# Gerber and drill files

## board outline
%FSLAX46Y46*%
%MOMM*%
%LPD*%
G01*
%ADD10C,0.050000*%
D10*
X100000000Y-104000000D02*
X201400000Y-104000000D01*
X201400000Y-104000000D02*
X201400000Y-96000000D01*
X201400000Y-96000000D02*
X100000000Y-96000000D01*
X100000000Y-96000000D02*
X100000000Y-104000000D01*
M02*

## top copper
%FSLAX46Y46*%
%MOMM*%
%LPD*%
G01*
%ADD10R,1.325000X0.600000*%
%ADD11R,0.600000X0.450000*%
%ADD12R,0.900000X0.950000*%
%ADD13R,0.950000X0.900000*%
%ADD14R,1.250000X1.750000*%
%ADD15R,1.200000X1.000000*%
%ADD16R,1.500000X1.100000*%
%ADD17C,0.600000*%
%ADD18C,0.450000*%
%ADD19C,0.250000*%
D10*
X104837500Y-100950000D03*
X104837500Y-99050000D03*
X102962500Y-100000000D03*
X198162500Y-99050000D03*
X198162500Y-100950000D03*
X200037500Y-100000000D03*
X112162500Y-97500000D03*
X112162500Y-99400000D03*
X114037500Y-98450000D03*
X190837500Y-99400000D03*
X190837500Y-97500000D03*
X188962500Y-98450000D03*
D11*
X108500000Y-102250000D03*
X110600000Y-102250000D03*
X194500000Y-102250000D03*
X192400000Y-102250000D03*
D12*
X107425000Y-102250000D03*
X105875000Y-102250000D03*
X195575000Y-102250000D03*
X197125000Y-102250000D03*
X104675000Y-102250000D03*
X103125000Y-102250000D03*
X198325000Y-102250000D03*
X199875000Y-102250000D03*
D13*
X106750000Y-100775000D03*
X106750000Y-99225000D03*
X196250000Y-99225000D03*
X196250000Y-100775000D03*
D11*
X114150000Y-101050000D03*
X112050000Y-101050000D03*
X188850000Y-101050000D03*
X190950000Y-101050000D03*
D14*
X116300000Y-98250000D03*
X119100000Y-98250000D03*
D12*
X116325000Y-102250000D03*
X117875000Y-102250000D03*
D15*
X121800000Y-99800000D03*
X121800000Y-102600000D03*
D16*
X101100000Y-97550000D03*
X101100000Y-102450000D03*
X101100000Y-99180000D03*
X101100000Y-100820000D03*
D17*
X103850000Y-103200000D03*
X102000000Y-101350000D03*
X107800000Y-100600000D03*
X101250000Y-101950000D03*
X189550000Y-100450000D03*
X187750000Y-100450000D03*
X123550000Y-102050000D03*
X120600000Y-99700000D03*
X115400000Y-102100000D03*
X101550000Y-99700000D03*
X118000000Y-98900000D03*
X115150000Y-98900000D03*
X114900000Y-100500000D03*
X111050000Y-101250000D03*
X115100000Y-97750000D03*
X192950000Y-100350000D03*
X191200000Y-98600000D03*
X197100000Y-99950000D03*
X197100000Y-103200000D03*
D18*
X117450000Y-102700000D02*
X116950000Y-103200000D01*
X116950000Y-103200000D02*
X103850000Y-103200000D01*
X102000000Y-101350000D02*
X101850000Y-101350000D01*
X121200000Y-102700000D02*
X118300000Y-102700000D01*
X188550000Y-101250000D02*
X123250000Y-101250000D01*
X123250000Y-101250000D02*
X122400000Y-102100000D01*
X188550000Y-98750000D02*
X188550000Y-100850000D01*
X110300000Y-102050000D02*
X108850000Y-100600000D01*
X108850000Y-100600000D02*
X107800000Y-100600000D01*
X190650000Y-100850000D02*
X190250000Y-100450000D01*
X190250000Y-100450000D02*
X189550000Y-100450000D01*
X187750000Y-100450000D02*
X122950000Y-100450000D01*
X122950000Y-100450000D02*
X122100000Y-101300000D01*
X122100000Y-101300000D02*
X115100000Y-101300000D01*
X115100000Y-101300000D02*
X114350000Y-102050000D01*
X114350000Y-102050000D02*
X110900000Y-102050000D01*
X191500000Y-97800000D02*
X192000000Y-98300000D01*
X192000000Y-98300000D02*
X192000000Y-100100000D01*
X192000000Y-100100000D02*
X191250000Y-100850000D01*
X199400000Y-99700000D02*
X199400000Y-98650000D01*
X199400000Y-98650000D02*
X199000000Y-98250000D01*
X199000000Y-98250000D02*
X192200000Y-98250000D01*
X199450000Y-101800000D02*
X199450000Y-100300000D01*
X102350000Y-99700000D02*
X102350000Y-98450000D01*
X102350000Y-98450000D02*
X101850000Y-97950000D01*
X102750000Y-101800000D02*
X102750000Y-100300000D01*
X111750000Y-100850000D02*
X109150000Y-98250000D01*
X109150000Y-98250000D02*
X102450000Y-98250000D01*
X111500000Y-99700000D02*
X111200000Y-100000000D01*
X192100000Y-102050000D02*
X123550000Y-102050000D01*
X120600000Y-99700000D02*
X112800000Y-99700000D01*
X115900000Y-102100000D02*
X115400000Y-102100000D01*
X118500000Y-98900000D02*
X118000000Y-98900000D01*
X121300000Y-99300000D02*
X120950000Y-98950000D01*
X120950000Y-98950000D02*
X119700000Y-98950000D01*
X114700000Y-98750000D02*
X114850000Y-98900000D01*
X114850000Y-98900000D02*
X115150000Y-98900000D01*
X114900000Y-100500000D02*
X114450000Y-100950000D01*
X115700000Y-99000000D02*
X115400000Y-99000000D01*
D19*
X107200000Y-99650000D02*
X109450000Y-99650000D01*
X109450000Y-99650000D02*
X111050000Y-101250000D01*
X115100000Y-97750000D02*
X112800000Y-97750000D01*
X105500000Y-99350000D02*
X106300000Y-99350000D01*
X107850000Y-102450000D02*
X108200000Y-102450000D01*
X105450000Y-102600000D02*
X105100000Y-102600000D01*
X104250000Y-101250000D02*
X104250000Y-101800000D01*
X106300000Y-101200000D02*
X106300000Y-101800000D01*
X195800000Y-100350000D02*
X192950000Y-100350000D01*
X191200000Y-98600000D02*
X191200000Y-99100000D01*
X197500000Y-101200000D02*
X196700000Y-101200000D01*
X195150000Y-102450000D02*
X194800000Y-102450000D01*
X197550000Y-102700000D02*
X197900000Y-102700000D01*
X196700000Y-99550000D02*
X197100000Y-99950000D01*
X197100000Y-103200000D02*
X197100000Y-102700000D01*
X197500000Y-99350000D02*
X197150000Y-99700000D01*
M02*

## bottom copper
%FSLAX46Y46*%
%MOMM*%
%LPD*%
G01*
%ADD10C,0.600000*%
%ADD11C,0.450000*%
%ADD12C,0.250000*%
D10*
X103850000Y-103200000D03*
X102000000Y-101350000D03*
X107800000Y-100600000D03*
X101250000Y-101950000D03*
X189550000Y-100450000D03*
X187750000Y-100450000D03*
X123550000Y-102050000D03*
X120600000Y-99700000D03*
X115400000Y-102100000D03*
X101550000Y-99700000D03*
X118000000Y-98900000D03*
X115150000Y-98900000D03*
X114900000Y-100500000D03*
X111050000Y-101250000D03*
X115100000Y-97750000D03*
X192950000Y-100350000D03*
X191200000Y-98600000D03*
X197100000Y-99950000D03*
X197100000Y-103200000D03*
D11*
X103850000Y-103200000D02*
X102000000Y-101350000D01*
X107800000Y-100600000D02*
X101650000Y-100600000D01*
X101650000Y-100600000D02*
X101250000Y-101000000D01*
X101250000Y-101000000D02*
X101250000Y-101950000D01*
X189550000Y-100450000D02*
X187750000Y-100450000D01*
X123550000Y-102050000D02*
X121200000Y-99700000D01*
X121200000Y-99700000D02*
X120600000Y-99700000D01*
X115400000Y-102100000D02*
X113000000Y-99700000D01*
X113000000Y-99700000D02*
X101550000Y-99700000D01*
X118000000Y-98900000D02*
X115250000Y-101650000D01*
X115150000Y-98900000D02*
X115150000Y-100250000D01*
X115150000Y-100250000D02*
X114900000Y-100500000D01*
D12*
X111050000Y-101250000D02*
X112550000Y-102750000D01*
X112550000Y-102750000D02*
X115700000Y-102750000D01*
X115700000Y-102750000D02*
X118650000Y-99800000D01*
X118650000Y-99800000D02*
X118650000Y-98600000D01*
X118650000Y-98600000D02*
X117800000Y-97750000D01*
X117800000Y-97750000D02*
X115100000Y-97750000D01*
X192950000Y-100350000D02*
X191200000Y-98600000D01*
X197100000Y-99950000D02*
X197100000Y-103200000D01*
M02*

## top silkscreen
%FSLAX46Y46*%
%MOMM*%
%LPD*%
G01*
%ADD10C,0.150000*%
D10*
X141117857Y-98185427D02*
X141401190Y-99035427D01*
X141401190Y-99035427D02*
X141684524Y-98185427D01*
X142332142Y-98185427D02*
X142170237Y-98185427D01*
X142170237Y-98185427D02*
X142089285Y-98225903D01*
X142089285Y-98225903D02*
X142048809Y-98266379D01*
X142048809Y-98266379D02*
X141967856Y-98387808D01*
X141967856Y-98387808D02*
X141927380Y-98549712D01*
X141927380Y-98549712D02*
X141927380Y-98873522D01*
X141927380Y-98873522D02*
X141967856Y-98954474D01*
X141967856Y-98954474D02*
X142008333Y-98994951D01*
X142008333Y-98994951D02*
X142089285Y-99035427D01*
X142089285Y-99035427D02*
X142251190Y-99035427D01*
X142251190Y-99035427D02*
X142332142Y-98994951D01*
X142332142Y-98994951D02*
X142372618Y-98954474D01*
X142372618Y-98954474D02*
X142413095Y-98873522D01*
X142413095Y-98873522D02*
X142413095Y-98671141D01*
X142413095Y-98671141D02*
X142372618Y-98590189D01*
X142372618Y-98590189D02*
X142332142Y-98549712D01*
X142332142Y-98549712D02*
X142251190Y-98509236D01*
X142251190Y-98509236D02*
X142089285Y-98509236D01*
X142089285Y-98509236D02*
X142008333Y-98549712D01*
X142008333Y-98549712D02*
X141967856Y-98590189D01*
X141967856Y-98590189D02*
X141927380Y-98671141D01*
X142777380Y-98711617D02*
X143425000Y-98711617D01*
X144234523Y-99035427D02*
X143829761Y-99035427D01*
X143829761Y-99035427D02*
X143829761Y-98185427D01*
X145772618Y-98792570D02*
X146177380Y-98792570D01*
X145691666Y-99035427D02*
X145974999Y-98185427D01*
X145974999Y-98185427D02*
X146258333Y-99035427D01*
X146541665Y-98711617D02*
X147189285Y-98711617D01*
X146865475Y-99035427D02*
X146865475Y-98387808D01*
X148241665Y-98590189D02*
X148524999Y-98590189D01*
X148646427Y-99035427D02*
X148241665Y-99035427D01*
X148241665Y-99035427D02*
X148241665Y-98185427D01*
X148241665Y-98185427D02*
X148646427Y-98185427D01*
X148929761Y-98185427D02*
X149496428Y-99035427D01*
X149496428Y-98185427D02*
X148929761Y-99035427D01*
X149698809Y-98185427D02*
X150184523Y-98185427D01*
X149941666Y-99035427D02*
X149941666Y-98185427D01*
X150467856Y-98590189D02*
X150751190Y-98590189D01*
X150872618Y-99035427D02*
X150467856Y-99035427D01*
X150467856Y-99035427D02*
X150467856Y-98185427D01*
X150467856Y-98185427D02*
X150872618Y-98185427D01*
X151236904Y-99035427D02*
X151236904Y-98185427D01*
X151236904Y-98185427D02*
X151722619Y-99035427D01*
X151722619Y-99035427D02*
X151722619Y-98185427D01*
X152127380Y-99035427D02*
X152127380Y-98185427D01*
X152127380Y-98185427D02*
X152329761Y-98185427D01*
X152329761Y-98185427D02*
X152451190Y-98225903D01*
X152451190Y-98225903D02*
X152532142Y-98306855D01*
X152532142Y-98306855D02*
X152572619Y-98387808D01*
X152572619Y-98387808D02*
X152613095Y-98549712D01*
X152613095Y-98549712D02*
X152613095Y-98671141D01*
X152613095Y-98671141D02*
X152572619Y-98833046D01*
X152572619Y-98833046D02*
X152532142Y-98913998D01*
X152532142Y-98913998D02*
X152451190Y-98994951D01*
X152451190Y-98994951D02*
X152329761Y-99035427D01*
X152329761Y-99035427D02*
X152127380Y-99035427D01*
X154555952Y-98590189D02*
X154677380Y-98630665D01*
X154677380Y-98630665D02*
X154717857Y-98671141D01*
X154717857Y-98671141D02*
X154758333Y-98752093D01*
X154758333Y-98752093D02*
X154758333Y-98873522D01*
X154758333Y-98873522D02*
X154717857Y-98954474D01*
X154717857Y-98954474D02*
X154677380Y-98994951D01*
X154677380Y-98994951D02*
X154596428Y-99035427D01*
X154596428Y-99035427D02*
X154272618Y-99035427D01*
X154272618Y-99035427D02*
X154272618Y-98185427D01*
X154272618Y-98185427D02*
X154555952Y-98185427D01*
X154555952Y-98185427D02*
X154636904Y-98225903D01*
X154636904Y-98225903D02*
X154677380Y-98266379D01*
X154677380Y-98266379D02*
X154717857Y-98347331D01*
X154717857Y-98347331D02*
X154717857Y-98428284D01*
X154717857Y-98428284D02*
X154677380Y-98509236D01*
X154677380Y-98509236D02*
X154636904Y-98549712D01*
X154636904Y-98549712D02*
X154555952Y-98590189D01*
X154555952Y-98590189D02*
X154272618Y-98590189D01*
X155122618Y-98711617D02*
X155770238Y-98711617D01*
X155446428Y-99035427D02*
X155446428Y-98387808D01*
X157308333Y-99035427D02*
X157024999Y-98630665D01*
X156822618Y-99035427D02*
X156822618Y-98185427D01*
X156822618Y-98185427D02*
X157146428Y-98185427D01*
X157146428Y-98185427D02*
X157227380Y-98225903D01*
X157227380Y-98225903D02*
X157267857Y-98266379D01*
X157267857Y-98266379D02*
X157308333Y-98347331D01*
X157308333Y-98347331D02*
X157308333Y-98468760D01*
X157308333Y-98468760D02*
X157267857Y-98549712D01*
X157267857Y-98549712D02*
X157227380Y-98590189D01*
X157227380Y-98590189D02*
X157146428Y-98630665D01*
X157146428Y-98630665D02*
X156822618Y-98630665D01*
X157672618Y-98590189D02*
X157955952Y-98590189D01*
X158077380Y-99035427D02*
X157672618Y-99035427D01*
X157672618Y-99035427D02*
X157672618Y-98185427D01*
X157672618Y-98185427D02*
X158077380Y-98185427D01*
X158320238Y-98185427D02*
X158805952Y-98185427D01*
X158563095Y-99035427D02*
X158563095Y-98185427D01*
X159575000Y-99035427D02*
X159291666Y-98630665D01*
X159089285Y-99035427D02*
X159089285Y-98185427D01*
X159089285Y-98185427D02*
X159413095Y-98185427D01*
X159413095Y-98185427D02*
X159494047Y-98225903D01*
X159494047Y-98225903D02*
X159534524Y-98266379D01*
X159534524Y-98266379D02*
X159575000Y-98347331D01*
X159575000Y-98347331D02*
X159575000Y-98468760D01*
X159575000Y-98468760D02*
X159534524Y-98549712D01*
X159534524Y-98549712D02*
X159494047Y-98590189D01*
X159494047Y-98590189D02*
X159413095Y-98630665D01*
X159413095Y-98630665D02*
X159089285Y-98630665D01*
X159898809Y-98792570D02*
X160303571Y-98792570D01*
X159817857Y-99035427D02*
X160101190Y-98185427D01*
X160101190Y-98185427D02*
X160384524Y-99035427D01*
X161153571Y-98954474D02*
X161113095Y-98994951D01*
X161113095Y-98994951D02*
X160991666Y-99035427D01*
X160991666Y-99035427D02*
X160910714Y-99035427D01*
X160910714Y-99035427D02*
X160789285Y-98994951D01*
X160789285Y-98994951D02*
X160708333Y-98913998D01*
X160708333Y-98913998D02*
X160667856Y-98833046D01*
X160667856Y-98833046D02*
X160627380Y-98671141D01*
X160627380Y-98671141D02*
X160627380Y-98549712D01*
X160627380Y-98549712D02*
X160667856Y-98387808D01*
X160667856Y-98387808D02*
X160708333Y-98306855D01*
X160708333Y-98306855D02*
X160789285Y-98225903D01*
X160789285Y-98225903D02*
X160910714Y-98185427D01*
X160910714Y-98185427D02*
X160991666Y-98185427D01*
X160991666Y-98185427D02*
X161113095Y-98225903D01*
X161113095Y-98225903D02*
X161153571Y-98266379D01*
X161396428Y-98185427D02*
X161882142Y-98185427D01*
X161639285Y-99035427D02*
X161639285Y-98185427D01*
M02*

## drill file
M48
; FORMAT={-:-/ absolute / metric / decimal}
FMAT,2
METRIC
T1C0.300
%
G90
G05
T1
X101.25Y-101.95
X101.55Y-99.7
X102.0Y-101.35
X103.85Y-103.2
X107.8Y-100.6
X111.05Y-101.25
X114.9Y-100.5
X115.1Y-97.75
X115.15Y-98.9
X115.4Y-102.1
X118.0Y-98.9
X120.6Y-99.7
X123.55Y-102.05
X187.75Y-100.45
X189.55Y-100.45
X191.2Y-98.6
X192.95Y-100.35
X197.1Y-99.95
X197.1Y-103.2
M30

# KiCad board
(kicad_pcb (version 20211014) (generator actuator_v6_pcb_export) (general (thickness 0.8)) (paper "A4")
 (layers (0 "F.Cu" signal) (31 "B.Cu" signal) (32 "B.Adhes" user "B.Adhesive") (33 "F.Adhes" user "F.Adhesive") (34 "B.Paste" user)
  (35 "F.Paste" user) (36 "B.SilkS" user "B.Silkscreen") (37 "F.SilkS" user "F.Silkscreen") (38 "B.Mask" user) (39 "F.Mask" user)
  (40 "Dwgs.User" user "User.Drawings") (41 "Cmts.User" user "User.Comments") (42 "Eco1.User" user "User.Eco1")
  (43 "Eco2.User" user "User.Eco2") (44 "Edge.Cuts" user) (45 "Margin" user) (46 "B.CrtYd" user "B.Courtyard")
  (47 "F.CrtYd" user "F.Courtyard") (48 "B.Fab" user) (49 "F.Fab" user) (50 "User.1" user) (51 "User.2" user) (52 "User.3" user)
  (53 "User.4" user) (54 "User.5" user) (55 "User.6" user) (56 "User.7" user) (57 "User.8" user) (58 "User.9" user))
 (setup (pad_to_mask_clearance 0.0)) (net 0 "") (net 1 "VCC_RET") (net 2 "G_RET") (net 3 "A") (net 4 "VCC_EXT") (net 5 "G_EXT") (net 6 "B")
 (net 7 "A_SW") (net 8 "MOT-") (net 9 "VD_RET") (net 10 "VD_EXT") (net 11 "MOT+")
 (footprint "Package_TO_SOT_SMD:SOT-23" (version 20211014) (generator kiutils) (layer "F.Cu") (at 103.9 100.0 180)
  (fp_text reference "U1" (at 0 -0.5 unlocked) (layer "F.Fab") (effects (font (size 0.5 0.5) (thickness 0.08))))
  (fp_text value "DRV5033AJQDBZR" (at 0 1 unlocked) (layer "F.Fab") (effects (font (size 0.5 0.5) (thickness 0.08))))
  (pad "1" smd rect (at -0.9375 -0.95 180) (size 1.325 0.6) (layers "F.Cu" "F.Mask" "F.Paste") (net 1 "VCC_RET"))
  (pad "2" smd rect (at -0.9375 0.95 180) (size 1.325 0.6) (layers "F.Cu" "F.Mask" "F.Paste") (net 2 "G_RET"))
  (pad "3" smd rect (at 0.9375 0.0 180) (size 1.325 0.6) (layers "F.Cu" "F.Mask" "F.Paste") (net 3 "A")))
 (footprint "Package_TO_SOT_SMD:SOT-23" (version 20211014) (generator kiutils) (layer "F.Cu") (at 199.1 100.0)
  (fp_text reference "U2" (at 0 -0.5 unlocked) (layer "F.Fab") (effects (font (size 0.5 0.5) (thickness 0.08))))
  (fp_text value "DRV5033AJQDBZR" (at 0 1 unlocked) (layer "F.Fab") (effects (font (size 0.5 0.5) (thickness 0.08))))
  (pad "1" smd rect (at -0.9375 -0.95) (size 1.325 0.6) (layers "F.Cu" "F.Mask" "F.Paste") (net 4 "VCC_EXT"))
  (pad "2" smd rect (at -0.9375 0.95) (size 1.325 0.6) (layers "F.Cu" "F.Mask" "F.Paste") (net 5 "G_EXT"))
  (pad "3" smd rect (at 0.9375 0.0) (size 1.325 0.6) (layers "F.Cu" "F.Mask" "F.Paste") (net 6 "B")))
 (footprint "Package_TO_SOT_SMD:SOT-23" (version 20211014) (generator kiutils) (layer "F.Cu") (at 113.1 98.45)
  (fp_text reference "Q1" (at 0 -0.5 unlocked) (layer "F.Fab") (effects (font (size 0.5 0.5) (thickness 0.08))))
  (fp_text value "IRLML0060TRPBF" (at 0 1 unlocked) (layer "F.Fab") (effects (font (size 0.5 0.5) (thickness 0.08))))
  (pad "1" smd rect (at -0.9375 -0.95) (size 1.325 0.6) (layers "F.Cu" "F.Mask" "F.Paste") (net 2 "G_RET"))
  (pad "2" smd rect (at -0.9375 0.95) (size 1.325 0.6) (layers "F.Cu" "F.Mask" "F.Paste") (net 3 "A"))
  (pad "3" smd rect (at 0.9375 0.0) (size 1.325 0.6) (layers "F.Cu" "F.Mask" "F.Paste") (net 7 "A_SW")))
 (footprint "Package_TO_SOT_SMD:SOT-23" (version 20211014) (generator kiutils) (layer "F.Cu") (at 189.9 98.45 180)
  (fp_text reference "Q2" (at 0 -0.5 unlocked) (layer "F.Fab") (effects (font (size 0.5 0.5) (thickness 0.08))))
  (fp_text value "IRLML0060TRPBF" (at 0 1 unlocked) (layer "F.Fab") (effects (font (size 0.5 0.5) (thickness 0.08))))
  (pad "1" smd rect (at -0.9375 -0.95 180) (size 1.325 0.6) (layers "F.Cu" "F.Mask" "F.Paste") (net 5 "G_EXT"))
  (pad "2" smd rect (at -0.9375 0.95 180) (size 1.325 0.6) (layers "F.Cu" "F.Mask" "F.Paste") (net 6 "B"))
  (pad "3" smd rect (at 0.9375 0.0 180) (size 1.325 0.6) (layers "F.Cu" "F.Mask" "F.Paste") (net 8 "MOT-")))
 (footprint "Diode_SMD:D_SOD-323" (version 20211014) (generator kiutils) (layer "F.Cu") (at 109.55 102.25)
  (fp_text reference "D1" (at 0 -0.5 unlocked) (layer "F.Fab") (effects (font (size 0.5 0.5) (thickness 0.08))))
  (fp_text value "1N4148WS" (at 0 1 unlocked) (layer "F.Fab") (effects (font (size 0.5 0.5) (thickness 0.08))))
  (pad "1" smd rect (at -1.05 0.0) (size 0.6 0.45) (layers "F.Cu" "F.Mask" "F.Paste") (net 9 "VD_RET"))
  (pad "2" smd rect (at 1.05 0.0) (size 0.6 0.45) (layers "F.Cu" "F.Mask" "F.Paste") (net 6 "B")))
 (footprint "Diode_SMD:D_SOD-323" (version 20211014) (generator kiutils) (layer "F.Cu") (at 193.45 102.25 180)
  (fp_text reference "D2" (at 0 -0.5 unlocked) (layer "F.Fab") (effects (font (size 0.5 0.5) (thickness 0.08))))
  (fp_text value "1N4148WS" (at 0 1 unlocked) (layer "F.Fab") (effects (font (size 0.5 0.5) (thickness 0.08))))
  (pad "1" smd rect (at -1.05 0.0 180) (size 0.6 0.45) (layers "F.Cu" "F.Mask" "F.Paste") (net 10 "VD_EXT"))
  (pad "2" smd rect (at 1.05 0.0 180) (size 0.6 0.45) (layers "F.Cu" "F.Mask" "F.Paste") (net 3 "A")))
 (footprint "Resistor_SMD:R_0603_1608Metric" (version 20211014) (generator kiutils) (layer "F.Cu") (at 106.65 102.25 180)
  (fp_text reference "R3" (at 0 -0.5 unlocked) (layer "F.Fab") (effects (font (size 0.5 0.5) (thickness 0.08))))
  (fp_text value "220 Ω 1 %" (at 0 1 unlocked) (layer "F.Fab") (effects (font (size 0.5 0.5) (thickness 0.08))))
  (pad "1" smd rect (at -0.775 0.0 180) (size 0.9 0.95) (layers "F.Cu" "F.Mask" "F.Paste") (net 9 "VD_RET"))
  (pad "2" smd rect (at 0.775 0.0 180) (size 0.9 0.95) (layers "F.Cu" "F.Mask" "F.Paste") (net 1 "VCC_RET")))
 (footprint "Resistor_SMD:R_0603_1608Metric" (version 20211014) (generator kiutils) (layer "F.Cu") (at 196.35 102.25)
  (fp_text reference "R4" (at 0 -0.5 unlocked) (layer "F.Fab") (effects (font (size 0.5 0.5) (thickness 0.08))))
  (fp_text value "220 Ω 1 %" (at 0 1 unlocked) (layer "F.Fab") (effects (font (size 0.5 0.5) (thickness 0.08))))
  (pad "1" smd rect (at -0.775 0.0) (size 0.9 0.95) (layers "F.Cu" "F.Mask" "F.Paste") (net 10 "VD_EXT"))
  (pad "2" smd rect (at 0.775 0.0) (size 0.9 0.95) (layers "F.Cu" "F.Mask" "F.Paste") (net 4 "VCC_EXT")))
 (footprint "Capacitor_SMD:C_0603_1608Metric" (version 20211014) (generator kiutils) (layer "F.Cu") (at 103.9 102.25 180)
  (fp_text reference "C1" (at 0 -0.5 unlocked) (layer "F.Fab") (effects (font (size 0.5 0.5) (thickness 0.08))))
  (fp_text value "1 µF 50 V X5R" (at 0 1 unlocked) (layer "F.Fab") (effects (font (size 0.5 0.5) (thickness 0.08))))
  (pad "1" smd rect (at -0.775 0.0 180) (size 0.9 0.95) (layers "F.Cu" "F.Mask" "F.Paste") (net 1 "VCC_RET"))
  (pad "2" smd rect (at 0.775 0.0 180) (size 0.9 0.95) (layers "F.Cu" "F.Mask" "F.Paste") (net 3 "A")))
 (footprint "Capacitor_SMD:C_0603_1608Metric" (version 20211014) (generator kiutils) (layer "F.Cu") (at 199.1 102.25)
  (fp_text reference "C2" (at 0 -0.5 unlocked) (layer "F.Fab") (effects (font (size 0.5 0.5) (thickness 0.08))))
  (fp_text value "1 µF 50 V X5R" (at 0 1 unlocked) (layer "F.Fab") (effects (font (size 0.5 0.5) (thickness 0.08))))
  (pad "1" smd rect (at -0.775 0.0) (size 0.9 0.95) (layers "F.Cu" "F.Mask" "F.Paste") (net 4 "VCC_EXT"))
  (pad "2" smd rect (at 0.775 0.0) (size 0.9 0.95) (layers "F.Cu" "F.Mask" "F.Paste") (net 6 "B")))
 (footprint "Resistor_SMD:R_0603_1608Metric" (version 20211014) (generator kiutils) (layer "F.Cu") (at 106.75 100.0 90)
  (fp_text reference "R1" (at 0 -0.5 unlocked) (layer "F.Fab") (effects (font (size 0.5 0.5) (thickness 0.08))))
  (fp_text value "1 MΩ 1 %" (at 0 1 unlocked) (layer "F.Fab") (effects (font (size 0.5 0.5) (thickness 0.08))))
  (pad "1" smd rect (at -0.775 0.0 90) (size 0.9 0.95) (layers "F.Cu" "F.Mask" "F.Paste") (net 1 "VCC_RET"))
  (pad "2" smd rect (at 0.775 0.0 90) (size 0.9 0.95) (layers "F.Cu" "F.Mask" "F.Paste") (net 2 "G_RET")))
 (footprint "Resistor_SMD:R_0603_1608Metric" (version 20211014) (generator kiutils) (layer "F.Cu") (at 196.25 100.0 270)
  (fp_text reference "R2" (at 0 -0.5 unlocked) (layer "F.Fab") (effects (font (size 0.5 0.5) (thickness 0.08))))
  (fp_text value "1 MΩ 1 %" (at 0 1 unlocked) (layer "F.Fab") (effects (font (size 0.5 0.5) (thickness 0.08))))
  (pad "1" smd rect (at -0.775 0.0 270) (size 0.9 0.95) (layers "F.Cu" "F.Mask" "F.Paste") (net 4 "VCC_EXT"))
  (pad "2" smd rect (at 0.775 0.0 270) (size 0.9 0.95) (layers "F.Cu" "F.Mask" "F.Paste") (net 5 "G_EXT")))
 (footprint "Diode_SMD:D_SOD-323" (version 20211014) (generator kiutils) (layer "F.Cu") (at 113.1 101.05 180)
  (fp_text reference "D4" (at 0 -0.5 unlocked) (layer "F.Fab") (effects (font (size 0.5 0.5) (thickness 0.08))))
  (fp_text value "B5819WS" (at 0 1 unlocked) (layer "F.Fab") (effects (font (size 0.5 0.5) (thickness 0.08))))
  (pad "1" smd rect (at -1.05 0.0 180) (size 0.6 0.45) (layers "F.Cu" "F.Mask" "F.Paste") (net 7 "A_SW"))
  (pad "2" smd rect (at 1.05 0.0 180) (size 0.6 0.45) (layers "F.Cu" "F.Mask" "F.Paste") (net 3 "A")))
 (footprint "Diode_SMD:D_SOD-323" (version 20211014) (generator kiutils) (layer "F.Cu") (at 189.9 101.05)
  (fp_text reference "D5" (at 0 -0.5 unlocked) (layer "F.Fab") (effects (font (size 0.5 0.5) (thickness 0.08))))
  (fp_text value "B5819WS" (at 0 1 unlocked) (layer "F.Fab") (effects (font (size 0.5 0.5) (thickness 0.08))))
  (pad "1" smd rect (at -1.05 0.0) (size 0.6 0.45) (layers "F.Cu" "F.Mask" "F.Paste") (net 8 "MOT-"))
  (pad "2" smd rect (at 1.05 0.0) (size 0.6 0.45) (layers "F.Cu" "F.Mask" "F.Paste") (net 6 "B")))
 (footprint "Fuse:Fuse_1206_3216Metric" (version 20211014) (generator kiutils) (layer "F.Cu") (at 117.7 98.25)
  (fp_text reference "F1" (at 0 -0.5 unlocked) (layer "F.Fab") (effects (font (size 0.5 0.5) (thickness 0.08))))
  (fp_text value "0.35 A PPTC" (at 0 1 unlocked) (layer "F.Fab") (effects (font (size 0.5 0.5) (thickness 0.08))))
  (pad "1" smd rect (at -1.4 0.0) (size 1.25 1.75) (layers "F.Cu" "F.Mask" "F.Paste") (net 7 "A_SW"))
  (pad "2" smd rect (at 1.4 0.0) (size 1.25 1.75) (layers "F.Cu" "F.Mask" "F.Paste") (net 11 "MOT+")))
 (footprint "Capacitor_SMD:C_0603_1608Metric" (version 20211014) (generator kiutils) (layer "F.Cu") (at 117.1 102.25)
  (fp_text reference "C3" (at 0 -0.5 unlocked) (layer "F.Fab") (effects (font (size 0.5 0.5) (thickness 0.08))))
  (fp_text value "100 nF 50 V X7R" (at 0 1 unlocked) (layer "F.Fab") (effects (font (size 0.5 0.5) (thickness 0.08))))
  (pad "1" smd rect (at -0.775 0.0) (size 0.9 0.95) (layers "F.Cu" "F.Mask" "F.Paste") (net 11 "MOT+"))
  (pad "2" smd rect (at 0.775 0.0) (size 0.9 0.95) (layers "F.Cu" "F.Mask" "F.Paste") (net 8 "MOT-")))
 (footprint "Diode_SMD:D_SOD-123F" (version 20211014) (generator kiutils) (layer "F.Cu") (at 121.8 101.2 270)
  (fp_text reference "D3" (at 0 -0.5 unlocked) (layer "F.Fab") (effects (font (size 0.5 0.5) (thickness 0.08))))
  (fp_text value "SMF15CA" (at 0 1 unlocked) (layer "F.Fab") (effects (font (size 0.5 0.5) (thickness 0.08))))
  (pad "1" smd rect (at -1.4 0.0 270) (size 1.0 1.2) (layers "F.Cu" "F.Mask" "F.Paste") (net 11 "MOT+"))
  (pad "2" smd rect (at 1.4 0.0 270) (size 1.0 1.2) (layers "F.Cu" "F.Mask" "F.Paste") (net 8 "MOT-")))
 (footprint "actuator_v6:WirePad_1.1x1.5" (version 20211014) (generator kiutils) (layer "F.Cu") (at 101.1 97.55)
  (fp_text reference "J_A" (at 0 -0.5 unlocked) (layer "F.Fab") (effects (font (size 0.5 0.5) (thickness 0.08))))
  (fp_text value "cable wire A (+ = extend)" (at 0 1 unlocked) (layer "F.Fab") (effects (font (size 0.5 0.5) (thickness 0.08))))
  (pad "1" smd rect (at 0.0 0.0) (size 1.5 1.1) (layers "F.Cu" "F.Mask") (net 3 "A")))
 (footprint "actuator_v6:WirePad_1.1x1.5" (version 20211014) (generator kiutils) (layer "F.Cu") (at 101.1 102.45)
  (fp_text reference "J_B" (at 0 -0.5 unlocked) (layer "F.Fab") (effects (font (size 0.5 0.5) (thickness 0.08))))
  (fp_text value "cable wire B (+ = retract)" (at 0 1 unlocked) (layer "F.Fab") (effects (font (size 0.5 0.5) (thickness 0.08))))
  (pad "1" smd rect (at 0.0 0.0) (size 1.5 1.1) (layers "F.Cu" "F.Mask") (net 6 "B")))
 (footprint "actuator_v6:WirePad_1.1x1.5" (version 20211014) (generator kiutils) (layer "F.Cu") (at 101.1 99.18)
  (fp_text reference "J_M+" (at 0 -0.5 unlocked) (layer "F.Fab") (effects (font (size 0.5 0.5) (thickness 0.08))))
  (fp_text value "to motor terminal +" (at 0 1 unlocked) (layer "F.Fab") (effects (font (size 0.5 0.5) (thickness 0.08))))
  (pad "1" smd rect (at 0.0 0.0) (size 1.5 1.1) (layers "F.Cu" "F.Mask") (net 11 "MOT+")))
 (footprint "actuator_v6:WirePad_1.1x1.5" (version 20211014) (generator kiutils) (layer "F.Cu") (at 101.1 100.82)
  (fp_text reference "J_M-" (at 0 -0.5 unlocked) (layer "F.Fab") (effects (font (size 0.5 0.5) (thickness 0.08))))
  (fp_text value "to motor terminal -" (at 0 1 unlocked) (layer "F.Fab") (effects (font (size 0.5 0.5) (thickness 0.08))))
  (pad "1" smd rect (at 0.0 0.0) (size 1.5 1.1) (layers "F.Cu" "F.Mask") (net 8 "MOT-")))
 (gr_line (start 100.0 104.0) (end 201.4 104.0) (layer "Edge.Cuts") (width 0.05))
 (gr_line (start 201.4 104.0) (end 201.4 96.0) (layer "Edge.Cuts") (width 0.05))
 (gr_line (start 201.4 96.0) (end 100.0 96.0) (layer "Edge.Cuts") (width 0.05))
 (gr_line (start 100.0 96.0) (end 100.0 104.0) (layer "Edge.Cuts") (width 0.05))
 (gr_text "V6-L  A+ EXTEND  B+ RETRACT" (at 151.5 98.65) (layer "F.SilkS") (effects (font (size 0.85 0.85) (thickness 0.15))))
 (segment (start 117.45 102.7) (end 116.95 103.2) (width 0.45) (layer "F.Cu") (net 8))
 (segment (start 116.95 103.2) (end 103.85 103.2) (width 0.45) (layer "F.Cu") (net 8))
 (segment (start 103.85 103.2) (end 102.0 101.35) (width 0.45) (layer "B.Cu") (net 8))
 (segment (start 102.0 101.35) (end 101.85 101.35) (width 0.45) (layer "F.Cu") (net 8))
 (segment (start 121.2 102.7) (end 118.3 102.7) (width 0.45) (layer "F.Cu") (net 8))
 (segment (start 188.55 101.25) (end 123.25 101.25) (width 0.45) (layer "F.Cu") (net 8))
 (segment (start 123.25 101.25) (end 122.4 102.1) (width 0.45) (layer "F.Cu") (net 8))
 (segment (start 188.55 98.75) (end 188.55 100.85) (width 0.45) (layer "F.Cu") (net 8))
 (segment (start 110.3 102.05) (end 108.85 100.6) (width 0.45) (layer "F.Cu") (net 6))
 (segment (start 108.85 100.6) (end 107.8 100.6) (width 0.45) (layer "F.Cu") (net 6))
 (segment (start 107.8 100.6) (end 101.65 100.6) (width 0.45) (layer "B.Cu") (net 6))
 (segment (start 101.65 100.6) (end 101.25 101.0) (width 0.45) (layer "B.Cu") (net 6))
 (segment (start 101.25 101.0) (end 101.25 101.95) (width 0.45) (layer "B.Cu") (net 6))
 (segment (start 190.65 100.85) (end 190.25 100.45) (width 0.45) (layer "F.Cu") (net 6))
 (segment (start 190.25 100.45) (end 189.55 100.45) (width 0.45) (layer "F.Cu") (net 6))
 (segment (start 189.55 100.45) (end 187.75 100.45) (width 0.45) (layer "B.Cu") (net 6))
 (segment (start 187.75 100.45) (end 122.95 100.45) (width 0.45) (layer "F.Cu") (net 6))
 (segment (start 122.95 100.45) (end 122.1 101.3) (width 0.45) (layer "F.Cu") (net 6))
 (segment (start 122.1 101.3) (end 115.1 101.3) (width 0.45) (layer "F.Cu") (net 6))
 (segment (start 115.1 101.3) (end 114.35 102.05) (width 0.45) (layer "F.Cu") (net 6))
 (segment (start 114.35 102.05) (end 110.9 102.05) (width 0.45) (layer "F.Cu") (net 6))
 (segment (start 191.5 97.8) (end 192.0 98.3) (width 0.45) (layer "F.Cu") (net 6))
 (segment (start 192.0 98.3) (end 192.0 100.1) (width 0.45) (layer "F.Cu") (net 6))
 (segment (start 192.0 100.1) (end 191.25 100.85) (width 0.45) (layer "F.Cu") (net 6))
 (segment (start 199.4 99.7) (end 199.4 98.65) (width 0.45) (layer "F.Cu") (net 6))
 (segment (start 199.4 98.65) (end 199.0 98.25) (width 0.45) (layer "F.Cu") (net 6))
 (segment (start 199.0 98.25) (end 192.2 98.25) (width 0.45) (layer "F.Cu") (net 6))
 (segment (start 199.45 101.8) (end 199.45 100.3) (width 0.45) (layer "F.Cu") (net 6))
 (segment (start 102.35 99.7) (end 102.35 98.45) (width 0.45) (layer "F.Cu") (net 3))
 (segment (start 102.35 98.45) (end 101.85 97.95) (width 0.45) (layer "F.Cu") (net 3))
 (segment (start 102.75 101.8) (end 102.75 100.3) (width 0.45) (layer "F.Cu") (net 3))
 (segment (start 111.75 100.85) (end 109.15 98.25) (width 0.45) (layer "F.Cu") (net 3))
 (segment (start 109.15 98.25) (end 102.45 98.25) (width 0.45) (layer "F.Cu") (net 3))
 (segment (start 111.5 99.7) (end 111.2 100.0) (width 0.45) (layer "F.Cu") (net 3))
 (segment (start 192.1 102.05) (end 123.55 102.05) (width 0.45) (layer "F.Cu") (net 3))
 (segment (start 123.55 102.05) (end 121.2 99.7) (width 0.45) (layer "B.Cu") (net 3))
 (segment (start 121.2 99.7) (end 120.6 99.7) (width 0.45) (layer "B.Cu") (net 3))
 (segment (start 120.6 99.7) (end 112.8 99.7) (width 0.45) (layer "F.Cu") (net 3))
 (segment (start 115.9 102.1) (end 115.4 102.1) (width 0.45) (layer "F.Cu") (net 11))
 (segment (start 115.4 102.1) (end 113.0 99.7) (width 0.45) (layer "B.Cu") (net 11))
 (segment (start 113.0 99.7) (end 101.55 99.7) (width 0.45) (layer "B.Cu") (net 11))
 (segment (start 118.5 98.9) (end 118.0 98.9) (width 0.45) (layer "F.Cu") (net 11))
 (segment (start 118.0 98.9) (end 115.25 101.65) (width 0.45) (layer "B.Cu") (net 11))
 (segment (start 121.3 99.3) (end 120.95 98.95) (width 0.45) (layer "F.Cu") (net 11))
 (segment (start 120.95 98.95) (end 119.7 98.95) (width 0.45) (layer "F.Cu") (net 11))
 (segment (start 114.7 98.75) (end 114.85 98.9) (width 0.45) (layer "F.Cu") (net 7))
 (segment (start 114.85 98.9) (end 115.15 98.9) (width 0.45) (layer "F.Cu") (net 7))
 (segment (start 115.15 98.9) (end 115.15 100.25) (width 0.45) (layer "B.Cu") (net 7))
 (segment (start 115.15 100.25) (end 114.9 100.5) (width 0.45) (layer "B.Cu") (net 7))
 (segment (start 114.9 100.5) (end 114.45 100.95) (width 0.45) (layer "F.Cu") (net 7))
 (segment (start 115.7 99.0) (end 115.4 99.0) (width 0.45) (layer "F.Cu") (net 7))
 (segment (start 107.2 99.65) (end 109.45 99.65) (width 0.25) (layer "F.Cu") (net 2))
 (segment (start 109.45 99.65) (end 111.05 101.25) (width 0.25) (layer "F.Cu") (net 2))
 (segment (start 111.05 101.25) (end 112.55 102.75) (width 0.25) (layer "B.Cu") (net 2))
 (segment (start 112.55 102.75) (end 115.7 102.75) (width 0.25) (layer "B.Cu") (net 2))
 (segment (start 115.7 102.75) (end 118.65 99.8) (width 0.25) (layer "B.Cu") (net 2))
 (segment (start 118.65 99.8) (end 118.65 98.6) (width 0.25) (layer "B.Cu") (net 2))
 (segment (start 118.65 98.6) (end 117.8 97.75) (width 0.25) (layer "B.Cu") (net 2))
 (segment (start 117.8 97.75) (end 115.1 97.75) (width 0.25) (layer "B.Cu") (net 2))
 (segment (start 115.1 97.75) (end 112.8 97.75) (width 0.25) (layer "F.Cu") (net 2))
 (segment (start 105.5 99.35) (end 106.3 99.35) (width 0.25) (layer "F.Cu") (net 2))
 (segment (start 107.85 102.45) (end 108.2 102.45) (width 0.25) (layer "F.Cu") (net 9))
 (segment (start 105.45 102.6) (end 105.1 102.6) (width 0.25) (layer "F.Cu") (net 1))
 (segment (start 104.25 101.25) (end 104.25 101.8) (width 0.25) (layer "F.Cu") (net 1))
 (segment (start 106.3 101.2) (end 106.3 101.8) (width 0.25) (layer "F.Cu") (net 1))
 (segment (start 195.8 100.35) (end 192.95 100.35) (width 0.25) (layer "F.Cu") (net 5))
 (segment (start 192.95 100.35) (end 191.2 98.6) (width 0.25) (layer "B.Cu") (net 5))
 (segment (start 191.2 98.6) (end 191.2 99.1) (width 0.25) (layer "F.Cu") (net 5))
 (segment (start 197.5 101.2) (end 196.7 101.2) (width 0.25) (layer "F.Cu") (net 5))
 (segment (start 195.15 102.45) (end 194.8 102.45) (width 0.25) (layer "F.Cu") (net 10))
 (segment (start 197.55 102.7) (end 197.9 102.7) (width 0.25) (layer "F.Cu") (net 4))
 (segment (start 196.7 99.55) (end 197.1 99.95) (width 0.25) (layer "F.Cu") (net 4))
 (segment (start 197.1 99.95) (end 197.1 103.2) (width 0.25) (layer "B.Cu") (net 4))
 (segment (start 197.1 103.2) (end 197.1 102.7) (width 0.25) (layer "F.Cu") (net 4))
 (segment (start 197.5 99.35) (end 197.15 99.7) (width 0.25) (layer "F.Cu") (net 4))
 (via (at 103.85 103.2) (size 0.6) (drill 0.3) (layers "F.Cu" "B.Cu") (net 8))
 (via (at 102.0 101.35) (size 0.6) (drill 0.3) (layers "F.Cu" "B.Cu") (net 8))
 (via (at 107.8 100.6) (size 0.6) (drill 0.3) (layers "F.Cu" "B.Cu") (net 6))
 (via (at 101.25 101.95) (size 0.6) (drill 0.3) (layers "F.Cu" "B.Cu") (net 6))
 (via (at 189.55 100.45) (size 0.6) (drill 0.3) (layers "F.Cu" "B.Cu") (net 6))
 (via (at 187.75 100.45) (size 0.6) (drill 0.3) (layers "F.Cu" "B.Cu") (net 6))
 (via (at 123.55 102.05) (size 0.6) (drill 0.3) (layers "F.Cu" "B.Cu") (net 3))
 (via (at 120.6 99.7) (size 0.6) (drill 0.3) (layers "F.Cu" "B.Cu") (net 3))
 (via (at 115.4 102.1) (size 0.6) (drill 0.3) (layers "F.Cu" "B.Cu") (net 11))
 (via (at 101.55 99.7) (size 0.6) (drill 0.3) (layers "F.Cu" "B.Cu") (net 11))
 (via (at 118.0 98.9) (size 0.6) (drill 0.3) (layers "F.Cu" "B.Cu") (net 11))
 (via (at 115.15 98.9) (size 0.6) (drill 0.3) (layers "F.Cu" "B.Cu") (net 7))
 (via (at 114.9 100.5) (size 0.6) (drill 0.3) (layers "F.Cu" "B.Cu") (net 7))
 (via (at 111.05 101.25) (size 0.6) (drill 0.3) (layers "F.Cu" "B.Cu") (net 2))
 (via (at 115.1 97.75) (size 0.6) (drill 0.3) (layers "F.Cu" "B.Cu") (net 2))
 (via (at 192.95 100.35) (size 0.6) (drill 0.3) (layers "F.Cu" "B.Cu") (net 5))
 (via (at 191.2 98.6) (size 0.6) (drill 0.3) (layers "F.Cu" "B.Cu") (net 5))
 (via (at 197.1 99.95) (size 0.6) (drill 0.3) (layers "F.Cu" "B.Cu") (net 4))
 (via (at 197.1 103.2) (size 0.6) (drill 0.3) (layers "F.Cu" "B.Cu") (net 4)))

